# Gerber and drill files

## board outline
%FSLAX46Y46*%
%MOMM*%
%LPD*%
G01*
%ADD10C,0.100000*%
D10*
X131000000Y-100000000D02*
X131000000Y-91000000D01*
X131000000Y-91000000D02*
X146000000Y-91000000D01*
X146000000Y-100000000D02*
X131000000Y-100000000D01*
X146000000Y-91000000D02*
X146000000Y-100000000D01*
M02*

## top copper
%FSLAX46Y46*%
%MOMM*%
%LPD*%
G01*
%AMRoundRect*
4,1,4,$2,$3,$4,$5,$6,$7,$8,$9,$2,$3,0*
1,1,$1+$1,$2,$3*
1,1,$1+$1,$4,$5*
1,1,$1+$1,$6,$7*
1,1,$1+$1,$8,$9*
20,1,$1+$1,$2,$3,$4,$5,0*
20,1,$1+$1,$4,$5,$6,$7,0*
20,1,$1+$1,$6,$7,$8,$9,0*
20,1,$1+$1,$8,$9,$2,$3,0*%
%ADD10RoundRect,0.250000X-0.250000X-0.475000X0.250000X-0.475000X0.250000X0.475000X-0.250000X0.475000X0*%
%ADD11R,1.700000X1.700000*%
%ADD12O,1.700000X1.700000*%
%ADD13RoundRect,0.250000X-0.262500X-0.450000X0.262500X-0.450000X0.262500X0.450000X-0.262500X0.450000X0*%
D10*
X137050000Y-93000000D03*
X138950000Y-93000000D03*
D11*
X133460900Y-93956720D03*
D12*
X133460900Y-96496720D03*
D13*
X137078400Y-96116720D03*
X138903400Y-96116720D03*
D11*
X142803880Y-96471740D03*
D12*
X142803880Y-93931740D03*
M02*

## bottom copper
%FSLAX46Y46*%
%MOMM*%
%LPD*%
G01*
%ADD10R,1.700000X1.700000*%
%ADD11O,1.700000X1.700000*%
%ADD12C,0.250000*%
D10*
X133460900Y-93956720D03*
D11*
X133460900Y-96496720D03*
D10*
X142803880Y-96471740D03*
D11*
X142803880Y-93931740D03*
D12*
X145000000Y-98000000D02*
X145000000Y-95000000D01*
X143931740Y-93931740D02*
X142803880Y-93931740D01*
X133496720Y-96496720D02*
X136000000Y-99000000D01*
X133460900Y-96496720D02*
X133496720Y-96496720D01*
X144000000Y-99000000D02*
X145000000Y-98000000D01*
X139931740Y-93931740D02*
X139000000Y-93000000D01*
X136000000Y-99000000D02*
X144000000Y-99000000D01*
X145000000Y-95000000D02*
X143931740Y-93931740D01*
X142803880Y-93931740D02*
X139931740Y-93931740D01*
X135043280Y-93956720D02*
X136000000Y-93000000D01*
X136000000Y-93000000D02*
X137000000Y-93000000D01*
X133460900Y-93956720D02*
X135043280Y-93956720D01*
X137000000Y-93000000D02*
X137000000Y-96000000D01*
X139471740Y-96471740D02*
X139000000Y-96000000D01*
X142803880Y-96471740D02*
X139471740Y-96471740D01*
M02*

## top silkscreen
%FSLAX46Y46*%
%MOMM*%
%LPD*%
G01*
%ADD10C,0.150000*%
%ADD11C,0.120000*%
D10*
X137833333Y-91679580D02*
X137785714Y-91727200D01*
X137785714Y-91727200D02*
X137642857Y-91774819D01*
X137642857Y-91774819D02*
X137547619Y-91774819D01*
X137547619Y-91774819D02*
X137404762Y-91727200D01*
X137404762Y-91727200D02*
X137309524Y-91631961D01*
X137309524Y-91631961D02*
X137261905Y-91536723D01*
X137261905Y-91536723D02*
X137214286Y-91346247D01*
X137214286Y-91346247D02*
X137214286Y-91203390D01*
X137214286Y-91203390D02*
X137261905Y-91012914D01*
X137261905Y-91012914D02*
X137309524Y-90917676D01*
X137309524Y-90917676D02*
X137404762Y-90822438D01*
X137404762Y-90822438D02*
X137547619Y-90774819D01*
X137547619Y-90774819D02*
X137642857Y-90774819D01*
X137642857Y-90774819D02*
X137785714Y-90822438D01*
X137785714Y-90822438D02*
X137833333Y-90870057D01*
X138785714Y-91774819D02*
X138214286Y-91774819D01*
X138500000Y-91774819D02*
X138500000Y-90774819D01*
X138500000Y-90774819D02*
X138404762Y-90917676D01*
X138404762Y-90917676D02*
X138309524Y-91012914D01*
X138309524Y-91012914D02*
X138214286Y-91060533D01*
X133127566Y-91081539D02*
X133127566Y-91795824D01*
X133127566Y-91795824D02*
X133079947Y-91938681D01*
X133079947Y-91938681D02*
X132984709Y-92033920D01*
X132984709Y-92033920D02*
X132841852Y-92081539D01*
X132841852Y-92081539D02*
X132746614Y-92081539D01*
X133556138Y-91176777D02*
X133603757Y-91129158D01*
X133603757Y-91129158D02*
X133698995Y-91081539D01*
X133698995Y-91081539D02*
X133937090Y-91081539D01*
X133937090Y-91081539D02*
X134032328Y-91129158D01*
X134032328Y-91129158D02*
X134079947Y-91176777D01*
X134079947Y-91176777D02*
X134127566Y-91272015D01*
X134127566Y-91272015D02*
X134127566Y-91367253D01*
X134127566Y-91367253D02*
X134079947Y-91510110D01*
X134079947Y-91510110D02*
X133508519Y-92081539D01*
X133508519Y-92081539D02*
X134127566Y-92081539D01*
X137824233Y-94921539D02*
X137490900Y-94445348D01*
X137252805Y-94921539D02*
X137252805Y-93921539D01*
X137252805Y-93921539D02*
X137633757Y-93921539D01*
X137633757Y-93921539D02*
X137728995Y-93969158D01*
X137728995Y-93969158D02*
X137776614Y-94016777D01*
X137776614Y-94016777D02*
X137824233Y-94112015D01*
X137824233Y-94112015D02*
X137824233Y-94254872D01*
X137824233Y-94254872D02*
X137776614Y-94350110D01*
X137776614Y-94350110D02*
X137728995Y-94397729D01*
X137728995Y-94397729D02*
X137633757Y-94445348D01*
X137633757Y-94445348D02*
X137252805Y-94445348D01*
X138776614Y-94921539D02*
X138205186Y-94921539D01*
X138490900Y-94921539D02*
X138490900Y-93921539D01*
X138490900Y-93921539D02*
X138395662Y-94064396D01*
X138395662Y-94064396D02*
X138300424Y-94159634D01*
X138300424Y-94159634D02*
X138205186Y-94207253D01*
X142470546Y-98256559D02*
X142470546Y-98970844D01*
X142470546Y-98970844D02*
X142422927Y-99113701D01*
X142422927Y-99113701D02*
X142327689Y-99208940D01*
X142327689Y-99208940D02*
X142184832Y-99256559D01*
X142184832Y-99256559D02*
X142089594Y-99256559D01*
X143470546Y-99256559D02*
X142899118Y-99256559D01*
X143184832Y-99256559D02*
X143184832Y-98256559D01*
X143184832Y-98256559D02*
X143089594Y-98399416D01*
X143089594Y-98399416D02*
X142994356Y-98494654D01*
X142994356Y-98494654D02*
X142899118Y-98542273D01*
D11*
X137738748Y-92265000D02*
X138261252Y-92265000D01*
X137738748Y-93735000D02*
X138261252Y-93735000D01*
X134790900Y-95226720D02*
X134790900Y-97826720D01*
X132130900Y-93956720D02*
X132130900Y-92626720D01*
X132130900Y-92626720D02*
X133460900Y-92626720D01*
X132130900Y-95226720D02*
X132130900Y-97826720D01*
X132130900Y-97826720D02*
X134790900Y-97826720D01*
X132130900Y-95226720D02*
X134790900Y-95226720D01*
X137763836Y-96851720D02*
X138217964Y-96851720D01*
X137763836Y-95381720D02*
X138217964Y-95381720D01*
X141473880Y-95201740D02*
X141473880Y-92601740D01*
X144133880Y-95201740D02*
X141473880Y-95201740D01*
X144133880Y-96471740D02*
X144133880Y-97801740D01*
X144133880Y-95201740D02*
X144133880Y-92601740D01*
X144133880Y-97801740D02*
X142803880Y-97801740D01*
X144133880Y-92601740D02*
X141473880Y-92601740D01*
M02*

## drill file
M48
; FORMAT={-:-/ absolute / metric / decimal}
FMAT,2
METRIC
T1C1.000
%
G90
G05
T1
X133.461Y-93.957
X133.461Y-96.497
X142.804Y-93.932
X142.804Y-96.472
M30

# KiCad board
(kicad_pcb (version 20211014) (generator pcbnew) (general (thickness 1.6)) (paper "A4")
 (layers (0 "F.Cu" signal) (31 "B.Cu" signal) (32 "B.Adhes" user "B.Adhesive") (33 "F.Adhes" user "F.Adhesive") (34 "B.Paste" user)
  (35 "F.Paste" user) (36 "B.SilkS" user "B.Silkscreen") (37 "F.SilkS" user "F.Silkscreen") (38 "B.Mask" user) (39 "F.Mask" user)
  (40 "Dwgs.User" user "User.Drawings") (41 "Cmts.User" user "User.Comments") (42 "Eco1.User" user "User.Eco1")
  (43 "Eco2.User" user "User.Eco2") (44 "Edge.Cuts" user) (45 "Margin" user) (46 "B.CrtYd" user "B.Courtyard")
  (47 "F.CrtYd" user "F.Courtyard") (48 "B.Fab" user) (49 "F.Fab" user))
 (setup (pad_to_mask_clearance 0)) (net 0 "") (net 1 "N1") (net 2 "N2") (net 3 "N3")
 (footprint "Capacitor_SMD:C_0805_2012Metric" (layer "F.Cu") (at 138 93)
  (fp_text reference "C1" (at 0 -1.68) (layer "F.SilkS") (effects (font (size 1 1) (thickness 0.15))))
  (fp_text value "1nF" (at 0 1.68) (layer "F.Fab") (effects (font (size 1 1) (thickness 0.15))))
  (fp_line (start -0.261252 -0.735) (end 0.261252 -0.735) (layer "F.SilkS") (width 0.12))
  (fp_line (start -0.261252 0.735) (end 0.261252 0.735) (layer "F.SilkS") (width 0.12))
  (pad "1" smd roundrect locked (at -0.95 0) (size 1 1.45) (layers "F.Cu" "F.Paste" "F.Mask") (roundrect_rratio 0.25) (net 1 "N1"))
  (pad "2" smd roundrect locked (at 0.95 0) (size 1 1.45) (layers "F.Cu" "F.Paste" "F.Mask") (roundrect_rratio 0.25) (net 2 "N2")))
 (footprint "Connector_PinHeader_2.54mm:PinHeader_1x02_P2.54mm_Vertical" (layer "F.Cu") (at 133.4609 93.95672)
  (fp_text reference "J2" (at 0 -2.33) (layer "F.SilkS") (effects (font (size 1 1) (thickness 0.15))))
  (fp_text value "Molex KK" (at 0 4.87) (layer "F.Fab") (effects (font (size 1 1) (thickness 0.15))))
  (fp_line (start 1.33 1.27) (end 1.33 3.87) (layer "F.SilkS") (width 0.12))
  (fp_line (start -1.33 0) (end -1.33 -1.33) (layer "F.SilkS") (width 0.12))
  (fp_line (start -1.33 -1.33) (end 0 -1.33) (layer "F.SilkS") (width 0.12))
  (fp_line (start -1.33 1.27) (end -1.33 3.87) (layer "F.SilkS") (width 0.12))
  (fp_line (start -1.33 3.87) (end 1.33 3.87) (layer "F.SilkS") (width 0.12))
  (fp_line (start -1.33 1.27) (end 1.33 1.27) (layer "F.SilkS") (width 0.12))
  (pad "1" thru_hole rect locked (at 0 0) (size 1.7 1.7) (drill 1) (layers *.Cu *.Mask) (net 1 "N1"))
  (pad "2" thru_hole oval locked (at 0 2.54) (size 1.7 1.7) (drill 1) (layers *.Cu *.Mask) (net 2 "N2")))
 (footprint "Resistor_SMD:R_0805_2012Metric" (layer "F.Cu") (at 137.9909 96.11672)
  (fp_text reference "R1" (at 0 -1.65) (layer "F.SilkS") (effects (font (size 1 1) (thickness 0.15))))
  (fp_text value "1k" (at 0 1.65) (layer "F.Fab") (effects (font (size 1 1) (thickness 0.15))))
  (fp_line (start -0.227064 0.735) (end 0.227064 0.735) (layer "F.SilkS") (width 0.12))
  (fp_line (start -0.227064 -0.735) (end 0.227064 -0.735) (layer "F.SilkS") (width 0.12))
  (pad "1" smd roundrect locked (at -0.9125 0) (size 1.025 1.4) (layers "F.Cu" "F.Paste" "F.Mask") (roundrect_rratio 0.243902) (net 1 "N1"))
  (pad "2" smd roundrect locked (at 0.9125 0) (size 1.025 1.4) (layers "F.Cu" "F.Paste" "F.Mask") (roundrect_rratio 0.243902) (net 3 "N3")))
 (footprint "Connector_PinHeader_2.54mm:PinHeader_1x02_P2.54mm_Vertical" (layer "F.Cu") (at 142.80388 96.47174 180)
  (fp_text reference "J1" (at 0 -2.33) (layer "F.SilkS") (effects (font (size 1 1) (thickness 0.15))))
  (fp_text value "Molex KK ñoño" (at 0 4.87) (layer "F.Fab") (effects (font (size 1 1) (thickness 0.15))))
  (fp_line (start 1.33 1.27) (end 1.33 3.87) (layer "F.SilkS") (width 0.12))
  (fp_line (start -1.33 1.27) (end 1.33 1.27) (layer "F.SilkS") (width 0.12))
  (fp_line (start -1.33 0) (end -1.33 -1.33) (layer "F.SilkS") (width 0.12))
  (fp_line (start -1.33 1.27) (end -1.33 3.87) (layer "F.SilkS") (width 0.12))
  (fp_line (start -1.33 -1.33) (end 0 -1.33) (layer "F.SilkS") (width 0.12))
  (fp_line (start -1.33 3.87) (end 1.33 3.87) (layer "F.SilkS") (width 0.12))
  (pad "1" thru_hole rect locked (at 0 0 180) (size 1.7 1.7) (drill 1) (layers *.Cu *.Mask) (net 3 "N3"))
  (pad "2" thru_hole oval locked (at 0 2.54 180) (size 1.7 1.7) (drill 1) (layers *.Cu *.Mask) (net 2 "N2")))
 (gr_line (start 131 100) (end 131 91) (layer "Edge.Cuts") (width 0.1))
 (gr_line (start 131 91) (end 146 91) (layer "Edge.Cuts") (width 0.1))
 (gr_line (start 146 100) (end 131 100) (layer "Edge.Cuts") (width 0.1))
 (gr_line (start 146 91) (end 146 100) (layer "Edge.Cuts") (width 0.1))
 (segment (start 145 98) (end 145 95) (width 0.25) (layer "B.Cu") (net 2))
 (segment (start 143.93174 93.93174) (end 142.80388 93.93174) (width 0.25) (layer "B.Cu") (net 2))
 (segment (start 133.49672 96.49672) (end 136 99) (width 0.25) (layer "B.Cu") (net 2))
 (segment (start 133.4609 96.49672) (end 133.49672 96.49672) (width 0.25) (layer "B.Cu") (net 2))
 (segment (start 144 99) (end 145 98) (width 0.25) (layer "B.Cu") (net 2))
 (segment (start 139.93174 93.93174) (end 139 93) (width 0.25) (layer "B.Cu") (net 2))
 (segment (start 136 99) (end 144 99) (width 0.25) (layer "B.Cu") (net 2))
 (segment (start 145 95) (end 143.93174 93.93174) (width 0.25) (layer "B.Cu") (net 2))
 (segment (start 142.80388 93.93174) (end 139.93174 93.93174) (width 0.25) (layer "B.Cu") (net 2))
 (segment (start 135.04328 93.95672) (end 136 93) (width 0.25) (layer "B.Cu") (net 1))
 (segment (start 136 93) (end 137 93) (width 0.25) (layer "B.Cu") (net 1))
 (segment (start 133.4609 93.95672) (end 135.04328 93.95672) (width 0.25) (layer "B.Cu") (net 1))
 (segment (start 137 93) (end 137 96) (width 0.25) (layer "B.Cu") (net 1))
 (segment (start 139.47174 96.47174) (end 139 96) (width 0.25) (layer "B.Cu") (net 3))
 (segment (start 142.80388 96.47174) (end 139.47174 96.47174) (width 0.25) (layer "B.Cu") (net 3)))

